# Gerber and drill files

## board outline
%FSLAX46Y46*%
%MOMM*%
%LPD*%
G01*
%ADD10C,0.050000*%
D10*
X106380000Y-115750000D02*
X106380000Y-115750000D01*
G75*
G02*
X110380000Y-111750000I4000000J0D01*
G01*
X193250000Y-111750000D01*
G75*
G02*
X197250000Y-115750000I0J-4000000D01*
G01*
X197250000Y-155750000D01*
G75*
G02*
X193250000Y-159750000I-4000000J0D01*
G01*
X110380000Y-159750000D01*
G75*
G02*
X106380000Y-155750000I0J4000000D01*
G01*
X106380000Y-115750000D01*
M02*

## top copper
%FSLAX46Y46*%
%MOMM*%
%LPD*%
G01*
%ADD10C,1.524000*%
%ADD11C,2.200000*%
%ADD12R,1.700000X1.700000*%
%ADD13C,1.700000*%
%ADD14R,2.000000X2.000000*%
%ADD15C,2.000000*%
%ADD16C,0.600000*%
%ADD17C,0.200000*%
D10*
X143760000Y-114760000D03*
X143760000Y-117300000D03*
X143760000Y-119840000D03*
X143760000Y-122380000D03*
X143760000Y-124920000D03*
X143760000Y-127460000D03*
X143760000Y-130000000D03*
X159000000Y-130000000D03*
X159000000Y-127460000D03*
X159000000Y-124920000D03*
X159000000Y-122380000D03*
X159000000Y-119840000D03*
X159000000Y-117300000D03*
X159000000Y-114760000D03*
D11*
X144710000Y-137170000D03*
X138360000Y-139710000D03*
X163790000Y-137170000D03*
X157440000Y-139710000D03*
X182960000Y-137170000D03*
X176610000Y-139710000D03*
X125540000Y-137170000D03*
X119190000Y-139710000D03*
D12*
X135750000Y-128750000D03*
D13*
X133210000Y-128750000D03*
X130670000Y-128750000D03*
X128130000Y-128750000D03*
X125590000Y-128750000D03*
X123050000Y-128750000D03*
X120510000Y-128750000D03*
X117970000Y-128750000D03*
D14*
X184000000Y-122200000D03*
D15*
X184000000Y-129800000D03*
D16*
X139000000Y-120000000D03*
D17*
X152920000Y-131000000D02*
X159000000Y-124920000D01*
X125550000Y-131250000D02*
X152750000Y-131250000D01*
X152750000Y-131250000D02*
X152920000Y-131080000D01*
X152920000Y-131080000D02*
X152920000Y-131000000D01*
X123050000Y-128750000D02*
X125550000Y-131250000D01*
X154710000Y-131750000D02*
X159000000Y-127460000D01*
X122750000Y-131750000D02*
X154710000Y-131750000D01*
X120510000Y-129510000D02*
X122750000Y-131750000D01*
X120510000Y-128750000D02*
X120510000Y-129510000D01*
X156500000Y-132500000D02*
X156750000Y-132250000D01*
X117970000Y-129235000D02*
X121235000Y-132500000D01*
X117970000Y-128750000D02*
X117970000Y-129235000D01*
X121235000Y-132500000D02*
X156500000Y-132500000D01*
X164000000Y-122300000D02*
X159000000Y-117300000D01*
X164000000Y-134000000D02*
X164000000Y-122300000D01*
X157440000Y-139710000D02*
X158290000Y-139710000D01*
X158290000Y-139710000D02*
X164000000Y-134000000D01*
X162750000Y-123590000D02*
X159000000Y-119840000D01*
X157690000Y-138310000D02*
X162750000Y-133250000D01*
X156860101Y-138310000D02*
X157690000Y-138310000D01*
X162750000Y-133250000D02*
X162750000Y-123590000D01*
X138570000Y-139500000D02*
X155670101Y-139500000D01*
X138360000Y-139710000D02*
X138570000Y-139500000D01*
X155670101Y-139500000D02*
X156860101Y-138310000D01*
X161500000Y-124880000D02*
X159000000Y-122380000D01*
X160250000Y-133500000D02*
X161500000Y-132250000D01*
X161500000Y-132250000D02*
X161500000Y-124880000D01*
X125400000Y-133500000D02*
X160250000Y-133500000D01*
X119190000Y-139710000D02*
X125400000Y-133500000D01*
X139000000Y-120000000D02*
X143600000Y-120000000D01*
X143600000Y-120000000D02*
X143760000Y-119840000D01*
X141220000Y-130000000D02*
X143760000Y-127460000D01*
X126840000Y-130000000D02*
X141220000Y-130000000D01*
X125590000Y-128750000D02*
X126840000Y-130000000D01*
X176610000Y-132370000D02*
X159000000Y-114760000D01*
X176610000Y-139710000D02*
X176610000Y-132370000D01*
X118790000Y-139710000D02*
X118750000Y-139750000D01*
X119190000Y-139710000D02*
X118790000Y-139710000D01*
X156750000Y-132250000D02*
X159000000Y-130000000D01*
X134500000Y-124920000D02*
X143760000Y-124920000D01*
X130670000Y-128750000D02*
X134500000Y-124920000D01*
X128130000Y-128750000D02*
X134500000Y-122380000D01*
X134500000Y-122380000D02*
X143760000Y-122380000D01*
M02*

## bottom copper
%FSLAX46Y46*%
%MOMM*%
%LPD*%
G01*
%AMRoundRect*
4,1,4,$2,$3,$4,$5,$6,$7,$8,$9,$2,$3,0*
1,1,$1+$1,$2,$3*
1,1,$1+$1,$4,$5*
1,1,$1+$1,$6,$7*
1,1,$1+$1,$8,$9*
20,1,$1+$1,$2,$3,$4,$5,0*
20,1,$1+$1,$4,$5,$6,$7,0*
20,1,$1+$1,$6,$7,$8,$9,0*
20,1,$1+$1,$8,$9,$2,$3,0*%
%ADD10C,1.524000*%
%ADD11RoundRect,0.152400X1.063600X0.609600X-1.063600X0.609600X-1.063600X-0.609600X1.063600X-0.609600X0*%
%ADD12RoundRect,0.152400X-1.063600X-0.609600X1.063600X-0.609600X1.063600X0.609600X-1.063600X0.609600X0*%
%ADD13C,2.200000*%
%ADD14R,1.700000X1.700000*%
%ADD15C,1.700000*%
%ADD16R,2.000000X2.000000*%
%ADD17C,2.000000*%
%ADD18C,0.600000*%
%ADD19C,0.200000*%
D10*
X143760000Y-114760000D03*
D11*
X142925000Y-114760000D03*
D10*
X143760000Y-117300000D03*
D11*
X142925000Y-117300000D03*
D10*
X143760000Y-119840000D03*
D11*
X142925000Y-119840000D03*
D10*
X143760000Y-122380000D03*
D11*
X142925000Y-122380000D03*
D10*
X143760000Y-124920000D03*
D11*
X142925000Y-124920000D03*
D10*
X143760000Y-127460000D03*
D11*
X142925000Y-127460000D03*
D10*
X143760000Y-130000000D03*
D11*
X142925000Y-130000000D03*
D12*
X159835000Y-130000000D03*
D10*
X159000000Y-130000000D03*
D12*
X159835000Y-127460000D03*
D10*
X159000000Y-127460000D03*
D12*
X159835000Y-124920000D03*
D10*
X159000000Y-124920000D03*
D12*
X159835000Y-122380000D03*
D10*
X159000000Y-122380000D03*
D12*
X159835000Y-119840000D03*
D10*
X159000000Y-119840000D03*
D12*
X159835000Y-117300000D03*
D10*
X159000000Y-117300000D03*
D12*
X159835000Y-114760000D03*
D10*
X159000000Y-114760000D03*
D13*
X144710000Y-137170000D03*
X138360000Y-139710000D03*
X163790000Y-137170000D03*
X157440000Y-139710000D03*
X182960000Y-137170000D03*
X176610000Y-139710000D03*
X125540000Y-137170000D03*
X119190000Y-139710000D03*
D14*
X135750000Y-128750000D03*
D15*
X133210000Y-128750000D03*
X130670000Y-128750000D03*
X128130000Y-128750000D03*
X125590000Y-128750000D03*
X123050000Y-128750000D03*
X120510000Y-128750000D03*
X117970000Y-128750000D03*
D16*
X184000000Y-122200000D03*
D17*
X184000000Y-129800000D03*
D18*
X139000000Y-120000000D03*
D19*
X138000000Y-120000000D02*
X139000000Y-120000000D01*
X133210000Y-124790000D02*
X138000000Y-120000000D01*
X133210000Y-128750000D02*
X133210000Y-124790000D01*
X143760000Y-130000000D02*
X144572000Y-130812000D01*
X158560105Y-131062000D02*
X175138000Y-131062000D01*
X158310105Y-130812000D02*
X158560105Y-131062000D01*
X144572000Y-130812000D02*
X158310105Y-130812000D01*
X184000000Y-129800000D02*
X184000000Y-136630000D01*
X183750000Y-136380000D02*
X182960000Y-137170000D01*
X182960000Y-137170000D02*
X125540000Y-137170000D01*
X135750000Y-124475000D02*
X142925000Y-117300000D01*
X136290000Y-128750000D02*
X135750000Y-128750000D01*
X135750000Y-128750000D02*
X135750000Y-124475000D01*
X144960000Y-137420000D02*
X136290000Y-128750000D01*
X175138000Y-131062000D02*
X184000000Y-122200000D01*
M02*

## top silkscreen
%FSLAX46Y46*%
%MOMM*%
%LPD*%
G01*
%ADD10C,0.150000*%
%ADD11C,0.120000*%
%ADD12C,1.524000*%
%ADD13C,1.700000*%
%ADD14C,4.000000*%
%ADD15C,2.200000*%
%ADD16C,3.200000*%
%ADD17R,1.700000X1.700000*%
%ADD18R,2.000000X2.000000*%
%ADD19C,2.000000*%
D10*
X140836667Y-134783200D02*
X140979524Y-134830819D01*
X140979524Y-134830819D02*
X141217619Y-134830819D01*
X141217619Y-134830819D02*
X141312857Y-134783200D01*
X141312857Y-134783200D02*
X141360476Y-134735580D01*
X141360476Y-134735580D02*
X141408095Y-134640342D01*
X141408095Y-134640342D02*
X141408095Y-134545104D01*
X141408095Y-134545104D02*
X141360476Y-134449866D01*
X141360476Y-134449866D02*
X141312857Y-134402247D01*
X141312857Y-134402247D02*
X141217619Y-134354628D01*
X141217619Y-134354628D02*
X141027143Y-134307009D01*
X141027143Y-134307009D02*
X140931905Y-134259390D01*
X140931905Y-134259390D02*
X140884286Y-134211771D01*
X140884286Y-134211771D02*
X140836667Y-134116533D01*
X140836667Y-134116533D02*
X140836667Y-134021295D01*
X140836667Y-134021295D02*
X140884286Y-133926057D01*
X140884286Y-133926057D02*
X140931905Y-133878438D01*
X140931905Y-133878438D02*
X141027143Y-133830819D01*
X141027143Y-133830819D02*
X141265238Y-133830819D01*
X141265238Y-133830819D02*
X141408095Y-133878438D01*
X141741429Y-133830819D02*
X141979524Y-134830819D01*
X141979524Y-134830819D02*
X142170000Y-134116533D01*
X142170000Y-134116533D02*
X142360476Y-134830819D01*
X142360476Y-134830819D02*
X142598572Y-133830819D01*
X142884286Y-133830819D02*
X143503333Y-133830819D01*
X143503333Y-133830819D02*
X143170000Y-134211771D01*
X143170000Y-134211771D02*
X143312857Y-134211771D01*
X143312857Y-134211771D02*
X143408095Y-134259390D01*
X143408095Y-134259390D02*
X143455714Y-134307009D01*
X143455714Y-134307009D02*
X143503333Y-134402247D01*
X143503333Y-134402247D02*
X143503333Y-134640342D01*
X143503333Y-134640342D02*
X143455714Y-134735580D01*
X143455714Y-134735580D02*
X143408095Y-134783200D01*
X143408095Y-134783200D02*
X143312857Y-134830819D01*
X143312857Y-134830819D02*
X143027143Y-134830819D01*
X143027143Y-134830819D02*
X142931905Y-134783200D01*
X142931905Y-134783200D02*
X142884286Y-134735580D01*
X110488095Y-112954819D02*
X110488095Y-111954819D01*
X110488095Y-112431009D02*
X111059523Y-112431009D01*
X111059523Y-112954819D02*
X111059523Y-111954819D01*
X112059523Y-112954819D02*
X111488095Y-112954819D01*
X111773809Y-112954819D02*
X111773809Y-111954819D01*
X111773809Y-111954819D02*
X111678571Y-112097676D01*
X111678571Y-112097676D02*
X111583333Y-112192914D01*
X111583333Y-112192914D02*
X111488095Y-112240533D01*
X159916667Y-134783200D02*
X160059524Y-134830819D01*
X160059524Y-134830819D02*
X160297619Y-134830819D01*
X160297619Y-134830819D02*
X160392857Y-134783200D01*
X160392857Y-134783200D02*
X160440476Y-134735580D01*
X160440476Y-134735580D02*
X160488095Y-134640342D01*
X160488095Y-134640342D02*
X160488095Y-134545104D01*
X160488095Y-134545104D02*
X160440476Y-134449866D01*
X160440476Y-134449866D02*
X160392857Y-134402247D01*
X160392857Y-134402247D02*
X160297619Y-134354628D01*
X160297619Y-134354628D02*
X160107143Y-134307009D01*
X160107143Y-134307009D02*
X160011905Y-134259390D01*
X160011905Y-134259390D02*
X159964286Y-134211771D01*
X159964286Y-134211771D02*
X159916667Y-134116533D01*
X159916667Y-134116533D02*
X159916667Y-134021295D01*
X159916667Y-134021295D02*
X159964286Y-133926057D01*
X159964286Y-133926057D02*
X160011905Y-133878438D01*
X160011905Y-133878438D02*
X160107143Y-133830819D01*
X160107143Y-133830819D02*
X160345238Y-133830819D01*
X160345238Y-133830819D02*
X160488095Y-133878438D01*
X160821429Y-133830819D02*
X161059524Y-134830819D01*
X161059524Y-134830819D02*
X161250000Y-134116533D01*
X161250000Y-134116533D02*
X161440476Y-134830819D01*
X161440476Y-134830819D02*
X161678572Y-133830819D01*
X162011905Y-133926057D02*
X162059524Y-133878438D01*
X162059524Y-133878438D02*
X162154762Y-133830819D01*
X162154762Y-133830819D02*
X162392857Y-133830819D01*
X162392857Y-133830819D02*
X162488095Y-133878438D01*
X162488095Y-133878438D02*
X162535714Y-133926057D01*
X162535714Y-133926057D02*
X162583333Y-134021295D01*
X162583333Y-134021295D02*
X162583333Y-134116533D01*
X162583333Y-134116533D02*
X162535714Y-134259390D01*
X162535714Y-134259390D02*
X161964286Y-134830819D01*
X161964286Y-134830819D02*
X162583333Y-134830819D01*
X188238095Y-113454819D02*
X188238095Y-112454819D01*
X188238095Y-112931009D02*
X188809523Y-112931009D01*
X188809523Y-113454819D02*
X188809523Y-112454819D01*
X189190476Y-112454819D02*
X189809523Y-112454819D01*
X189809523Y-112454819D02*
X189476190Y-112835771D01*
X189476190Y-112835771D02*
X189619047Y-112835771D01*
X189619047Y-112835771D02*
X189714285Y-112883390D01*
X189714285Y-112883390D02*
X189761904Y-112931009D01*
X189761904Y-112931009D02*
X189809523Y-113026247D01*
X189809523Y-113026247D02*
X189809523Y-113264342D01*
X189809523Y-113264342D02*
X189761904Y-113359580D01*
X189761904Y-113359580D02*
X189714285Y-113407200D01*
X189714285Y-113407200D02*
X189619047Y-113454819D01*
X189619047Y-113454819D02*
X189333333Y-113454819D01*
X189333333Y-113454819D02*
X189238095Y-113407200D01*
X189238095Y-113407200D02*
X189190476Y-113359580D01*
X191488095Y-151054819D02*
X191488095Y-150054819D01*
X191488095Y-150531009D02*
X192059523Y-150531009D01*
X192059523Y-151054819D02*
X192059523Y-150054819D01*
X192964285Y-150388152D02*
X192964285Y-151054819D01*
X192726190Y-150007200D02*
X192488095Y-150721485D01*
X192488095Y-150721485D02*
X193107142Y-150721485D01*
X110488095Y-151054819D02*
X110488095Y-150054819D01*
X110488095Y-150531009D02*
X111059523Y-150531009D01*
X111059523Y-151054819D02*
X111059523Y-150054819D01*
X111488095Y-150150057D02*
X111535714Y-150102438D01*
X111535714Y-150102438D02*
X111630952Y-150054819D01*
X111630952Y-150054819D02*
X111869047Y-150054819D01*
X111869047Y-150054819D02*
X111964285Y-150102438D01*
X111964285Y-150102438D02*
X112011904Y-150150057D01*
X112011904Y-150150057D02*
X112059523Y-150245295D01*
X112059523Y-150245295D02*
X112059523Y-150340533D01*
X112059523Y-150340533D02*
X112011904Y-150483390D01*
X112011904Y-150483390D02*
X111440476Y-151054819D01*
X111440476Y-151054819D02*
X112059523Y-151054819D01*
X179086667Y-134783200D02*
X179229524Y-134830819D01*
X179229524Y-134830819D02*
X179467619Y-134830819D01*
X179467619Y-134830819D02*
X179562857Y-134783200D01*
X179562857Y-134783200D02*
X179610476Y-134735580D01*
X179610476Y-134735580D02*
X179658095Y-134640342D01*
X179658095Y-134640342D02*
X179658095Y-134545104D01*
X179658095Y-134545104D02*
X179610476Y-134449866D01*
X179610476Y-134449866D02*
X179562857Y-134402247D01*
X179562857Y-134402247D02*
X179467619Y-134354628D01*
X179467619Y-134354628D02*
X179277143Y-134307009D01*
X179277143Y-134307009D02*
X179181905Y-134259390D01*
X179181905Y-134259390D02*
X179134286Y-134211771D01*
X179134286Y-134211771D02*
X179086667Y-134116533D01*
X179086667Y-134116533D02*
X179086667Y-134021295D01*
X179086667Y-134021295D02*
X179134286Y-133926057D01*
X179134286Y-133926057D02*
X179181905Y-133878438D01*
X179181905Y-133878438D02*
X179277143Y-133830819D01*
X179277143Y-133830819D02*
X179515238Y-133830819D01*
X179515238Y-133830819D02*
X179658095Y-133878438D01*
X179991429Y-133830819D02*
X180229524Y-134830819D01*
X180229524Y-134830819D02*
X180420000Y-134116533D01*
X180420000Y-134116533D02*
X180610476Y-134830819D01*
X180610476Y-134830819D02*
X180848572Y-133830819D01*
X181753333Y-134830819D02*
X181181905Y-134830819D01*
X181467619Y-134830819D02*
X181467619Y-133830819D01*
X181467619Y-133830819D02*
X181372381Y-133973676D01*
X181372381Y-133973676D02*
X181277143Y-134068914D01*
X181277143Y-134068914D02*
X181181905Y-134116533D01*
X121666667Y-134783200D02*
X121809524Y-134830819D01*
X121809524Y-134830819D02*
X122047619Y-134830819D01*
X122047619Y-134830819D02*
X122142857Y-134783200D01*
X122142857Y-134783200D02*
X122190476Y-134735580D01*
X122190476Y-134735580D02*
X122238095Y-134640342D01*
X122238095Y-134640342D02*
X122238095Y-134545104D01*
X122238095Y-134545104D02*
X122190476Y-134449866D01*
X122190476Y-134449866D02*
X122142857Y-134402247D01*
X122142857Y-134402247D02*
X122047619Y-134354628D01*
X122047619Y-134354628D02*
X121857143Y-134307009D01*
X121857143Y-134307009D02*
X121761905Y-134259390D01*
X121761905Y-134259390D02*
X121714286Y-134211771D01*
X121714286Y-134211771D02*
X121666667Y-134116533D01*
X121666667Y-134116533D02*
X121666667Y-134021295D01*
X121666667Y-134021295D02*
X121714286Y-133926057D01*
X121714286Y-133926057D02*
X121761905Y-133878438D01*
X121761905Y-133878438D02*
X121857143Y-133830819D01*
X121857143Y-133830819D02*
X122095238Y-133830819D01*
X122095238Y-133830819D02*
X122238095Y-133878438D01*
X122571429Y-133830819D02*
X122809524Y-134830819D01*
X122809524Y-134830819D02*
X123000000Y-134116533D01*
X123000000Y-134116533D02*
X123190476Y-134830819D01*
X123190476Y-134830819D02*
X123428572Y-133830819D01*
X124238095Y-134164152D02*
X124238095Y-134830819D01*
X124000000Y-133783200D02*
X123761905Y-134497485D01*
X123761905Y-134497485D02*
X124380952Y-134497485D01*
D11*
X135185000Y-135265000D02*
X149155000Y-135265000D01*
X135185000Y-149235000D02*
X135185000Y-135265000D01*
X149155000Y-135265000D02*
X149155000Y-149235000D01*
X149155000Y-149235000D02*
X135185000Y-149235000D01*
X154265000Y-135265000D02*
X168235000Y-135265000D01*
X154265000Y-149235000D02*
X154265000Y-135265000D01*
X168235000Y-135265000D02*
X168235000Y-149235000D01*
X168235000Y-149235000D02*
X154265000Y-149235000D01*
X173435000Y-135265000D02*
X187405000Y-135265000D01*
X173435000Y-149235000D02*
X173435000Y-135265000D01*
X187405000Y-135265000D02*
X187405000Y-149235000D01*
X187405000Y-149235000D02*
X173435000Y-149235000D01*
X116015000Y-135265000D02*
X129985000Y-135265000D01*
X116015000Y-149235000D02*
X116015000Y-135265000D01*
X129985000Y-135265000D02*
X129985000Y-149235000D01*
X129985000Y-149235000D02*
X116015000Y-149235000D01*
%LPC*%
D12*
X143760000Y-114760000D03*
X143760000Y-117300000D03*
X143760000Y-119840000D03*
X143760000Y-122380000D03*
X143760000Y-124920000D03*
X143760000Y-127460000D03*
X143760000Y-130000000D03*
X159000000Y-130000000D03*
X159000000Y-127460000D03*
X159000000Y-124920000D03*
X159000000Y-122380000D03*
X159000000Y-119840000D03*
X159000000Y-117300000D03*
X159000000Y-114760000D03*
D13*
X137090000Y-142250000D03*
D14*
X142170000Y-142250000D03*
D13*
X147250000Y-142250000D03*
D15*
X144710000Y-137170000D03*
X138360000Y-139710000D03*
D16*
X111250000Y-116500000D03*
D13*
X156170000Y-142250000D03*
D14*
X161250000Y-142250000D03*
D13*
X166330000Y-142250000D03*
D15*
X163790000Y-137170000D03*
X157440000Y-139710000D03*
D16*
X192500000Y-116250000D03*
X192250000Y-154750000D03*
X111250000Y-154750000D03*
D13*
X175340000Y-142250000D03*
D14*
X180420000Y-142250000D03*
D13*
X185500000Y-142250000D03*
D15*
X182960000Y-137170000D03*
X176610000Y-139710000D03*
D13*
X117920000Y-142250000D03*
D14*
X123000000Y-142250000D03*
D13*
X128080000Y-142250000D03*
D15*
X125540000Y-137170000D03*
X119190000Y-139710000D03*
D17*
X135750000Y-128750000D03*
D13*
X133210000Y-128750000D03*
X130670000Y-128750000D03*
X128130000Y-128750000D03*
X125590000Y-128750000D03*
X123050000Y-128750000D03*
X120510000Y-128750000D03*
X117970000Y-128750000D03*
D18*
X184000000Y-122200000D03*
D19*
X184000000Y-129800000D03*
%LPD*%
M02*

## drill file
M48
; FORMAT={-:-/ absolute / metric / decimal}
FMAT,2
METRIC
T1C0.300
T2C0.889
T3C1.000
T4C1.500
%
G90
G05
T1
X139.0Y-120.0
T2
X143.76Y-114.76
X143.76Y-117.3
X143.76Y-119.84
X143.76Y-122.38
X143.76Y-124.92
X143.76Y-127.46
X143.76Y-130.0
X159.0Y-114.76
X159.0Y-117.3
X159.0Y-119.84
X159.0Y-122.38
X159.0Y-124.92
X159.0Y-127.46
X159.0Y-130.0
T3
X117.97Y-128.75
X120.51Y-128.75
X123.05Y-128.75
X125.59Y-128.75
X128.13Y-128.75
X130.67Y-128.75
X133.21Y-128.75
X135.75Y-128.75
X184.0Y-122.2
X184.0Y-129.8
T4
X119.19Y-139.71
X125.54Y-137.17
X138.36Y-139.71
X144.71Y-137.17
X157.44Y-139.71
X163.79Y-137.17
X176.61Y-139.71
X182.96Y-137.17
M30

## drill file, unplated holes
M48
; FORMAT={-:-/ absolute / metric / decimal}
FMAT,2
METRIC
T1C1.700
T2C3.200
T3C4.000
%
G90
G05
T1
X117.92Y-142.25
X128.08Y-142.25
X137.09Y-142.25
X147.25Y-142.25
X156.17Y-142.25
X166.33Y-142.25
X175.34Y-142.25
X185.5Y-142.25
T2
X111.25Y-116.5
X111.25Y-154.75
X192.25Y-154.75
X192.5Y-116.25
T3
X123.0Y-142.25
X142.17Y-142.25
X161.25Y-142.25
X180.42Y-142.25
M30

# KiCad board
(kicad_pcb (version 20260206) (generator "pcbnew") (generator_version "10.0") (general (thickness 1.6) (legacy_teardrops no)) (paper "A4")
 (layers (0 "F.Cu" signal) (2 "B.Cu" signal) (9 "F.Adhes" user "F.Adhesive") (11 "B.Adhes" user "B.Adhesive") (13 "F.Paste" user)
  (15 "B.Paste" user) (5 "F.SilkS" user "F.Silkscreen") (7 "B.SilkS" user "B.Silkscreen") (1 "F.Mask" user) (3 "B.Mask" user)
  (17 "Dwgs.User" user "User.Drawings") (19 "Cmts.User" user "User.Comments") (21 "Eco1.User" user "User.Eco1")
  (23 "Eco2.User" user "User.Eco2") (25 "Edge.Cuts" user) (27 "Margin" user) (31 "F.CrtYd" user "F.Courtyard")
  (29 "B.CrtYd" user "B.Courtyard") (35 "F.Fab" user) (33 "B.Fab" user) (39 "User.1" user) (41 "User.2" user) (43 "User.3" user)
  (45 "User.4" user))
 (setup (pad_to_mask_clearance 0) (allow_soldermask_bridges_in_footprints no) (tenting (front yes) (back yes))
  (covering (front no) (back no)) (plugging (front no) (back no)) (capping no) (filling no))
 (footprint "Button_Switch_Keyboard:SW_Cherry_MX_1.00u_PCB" (layer "F.Cu") (at 144.71 137.17)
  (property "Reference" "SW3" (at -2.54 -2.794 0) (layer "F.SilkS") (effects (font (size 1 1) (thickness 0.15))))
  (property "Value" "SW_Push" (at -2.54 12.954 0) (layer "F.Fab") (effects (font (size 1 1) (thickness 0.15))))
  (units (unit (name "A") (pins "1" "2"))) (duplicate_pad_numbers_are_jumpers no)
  (fp_line (start -9.525 -1.905) (end 4.445 -1.905) (stroke (width 0.12) (type solid)) (layer "F.SilkS"))
  (fp_line (start -9.525 12.065) (end -9.525 -1.905) (stroke (width 0.12) (type solid)) (layer "F.SilkS"))
  (fp_line (start 4.445 -1.905) (end 4.445 12.065) (stroke (width 0.12) (type solid)) (layer "F.SilkS"))
  (fp_line (start 4.445 12.065) (end -9.525 12.065) (stroke (width 0.12) (type solid)) (layer "F.SilkS"))
  (pad "" np_thru_hole circle (at -7.62 5.08) (size 1.7 1.7) (drill 1.7) (layers "*.Cu" "*.Mask"))
  (pad "" np_thru_hole circle (at -2.54 5.08) (size 4 4) (drill 4) (layers "*.Cu" "*.Mask"))
  (pad "" np_thru_hole circle (at 2.54 5.08) (size 1.7 1.7) (drill 1.7) (layers "*.Cu" "*.Mask"))
  (pad "1" thru_hole circle (at 0 0) (size 2.2 2.2) (drill 1.5) (layers "*.Cu" "*.Mask") (remove_unused_layers no) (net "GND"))
  (pad "2" thru_hole circle (at -6.35 2.54) (size 2.2 2.2) (drill 1.5) (layers "*.Cu" "*.Mask") (remove_unused_layers no)
   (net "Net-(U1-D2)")))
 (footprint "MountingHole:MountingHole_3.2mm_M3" (layer "F.Cu") (at 111.25 116.5)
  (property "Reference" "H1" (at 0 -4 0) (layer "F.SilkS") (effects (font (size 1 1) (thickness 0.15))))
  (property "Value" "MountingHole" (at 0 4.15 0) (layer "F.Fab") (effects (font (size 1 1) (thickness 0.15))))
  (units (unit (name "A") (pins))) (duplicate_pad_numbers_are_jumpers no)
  (pad "" np_thru_hole circle (at 0 0) (size 3.2 3.2) (drill 3.2) (layers "*.Cu" "*.Mask")))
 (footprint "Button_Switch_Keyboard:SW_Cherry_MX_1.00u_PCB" (layer "F.Cu") (at 163.79 137.17)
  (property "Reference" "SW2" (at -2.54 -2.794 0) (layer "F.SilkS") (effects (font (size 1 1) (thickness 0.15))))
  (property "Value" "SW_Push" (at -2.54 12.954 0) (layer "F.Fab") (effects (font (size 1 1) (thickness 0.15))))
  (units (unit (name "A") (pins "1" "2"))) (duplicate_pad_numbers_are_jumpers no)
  (fp_line (start -9.525 -1.905) (end 4.445 -1.905) (stroke (width 0.12) (type solid)) (layer "F.SilkS"))
  (fp_line (start -9.525 12.065) (end -9.525 -1.905) (stroke (width 0.12) (type solid)) (layer "F.SilkS"))
  (fp_line (start 4.445 -1.905) (end 4.445 12.065) (stroke (width 0.12) (type solid)) (layer "F.SilkS"))
  (fp_line (start 4.445 12.065) (end -9.525 12.065) (stroke (width 0.12) (type solid)) (layer "F.SilkS"))
  (pad "" np_thru_hole circle (at -7.62 5.08) (size 1.7 1.7) (drill 1.7) (layers "*.Cu" "*.Mask"))
  (pad "" np_thru_hole circle (at -2.54 5.08) (size 4 4) (drill 4) (layers "*.Cu" "*.Mask"))
  (pad "" np_thru_hole circle (at 2.54 5.08) (size 1.7 1.7) (drill 1.7) (layers "*.Cu" "*.Mask"))
  (pad "1" thru_hole circle (at 0 0) (size 2.2 2.2) (drill 1.5) (layers "*.Cu" "*.Mask") (remove_unused_layers no) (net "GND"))
  (pad "2" thru_hole circle (at -6.35 2.54) (size 2.2 2.2) (drill 1.5) (layers "*.Cu" "*.Mask") (remove_unused_layers no)
   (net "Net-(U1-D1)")))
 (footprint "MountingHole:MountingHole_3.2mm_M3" (layer "F.Cu") (at 192.5 116.25)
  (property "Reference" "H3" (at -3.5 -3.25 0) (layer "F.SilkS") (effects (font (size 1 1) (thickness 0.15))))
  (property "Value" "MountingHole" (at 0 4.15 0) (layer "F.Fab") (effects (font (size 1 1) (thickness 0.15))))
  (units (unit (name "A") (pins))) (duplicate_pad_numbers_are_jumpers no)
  (pad "" np_thru_hole circle (at 0 0) (size 3.2 3.2) (drill 3.2) (layers "*.Cu" "*.Mask")))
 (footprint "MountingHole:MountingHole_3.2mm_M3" (layer "F.Cu") (at 192.25 154.75)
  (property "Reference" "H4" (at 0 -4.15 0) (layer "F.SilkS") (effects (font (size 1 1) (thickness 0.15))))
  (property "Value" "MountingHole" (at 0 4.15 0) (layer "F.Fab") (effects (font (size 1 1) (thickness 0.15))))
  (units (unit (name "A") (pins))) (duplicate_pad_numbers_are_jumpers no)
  (pad "" np_thru_hole circle (at 0 0) (size 3.2 3.2) (drill 3.2) (layers "*.Cu" "*.Mask")))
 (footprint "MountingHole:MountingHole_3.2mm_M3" (layer "F.Cu") (at 111.25 154.75)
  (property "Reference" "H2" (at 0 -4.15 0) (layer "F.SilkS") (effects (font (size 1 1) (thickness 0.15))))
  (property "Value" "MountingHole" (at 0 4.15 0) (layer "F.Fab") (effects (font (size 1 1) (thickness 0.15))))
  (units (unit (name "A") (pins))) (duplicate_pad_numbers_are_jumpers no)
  (pad "" np_thru_hole circle (at 0 0) (size 3.2 3.2) (drill 3.2) (layers "*.Cu" "*.Mask")))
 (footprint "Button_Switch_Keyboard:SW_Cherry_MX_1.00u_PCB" (layer "F.Cu") (at 182.96 137.17)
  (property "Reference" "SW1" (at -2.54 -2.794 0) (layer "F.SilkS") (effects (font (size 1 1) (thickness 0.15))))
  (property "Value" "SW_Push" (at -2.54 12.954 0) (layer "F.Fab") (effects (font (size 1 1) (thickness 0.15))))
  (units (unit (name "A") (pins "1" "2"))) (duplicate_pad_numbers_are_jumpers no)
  (fp_line (start -9.525 -1.905) (end 4.445 -1.905) (stroke (width 0.12) (type solid)) (layer "F.SilkS"))
  (fp_line (start -9.525 12.065) (end -9.525 -1.905) (stroke (width 0.12) (type solid)) (layer "F.SilkS"))
  (fp_line (start 4.445 -1.905) (end 4.445 12.065) (stroke (width 0.12) (type solid)) (layer "F.SilkS"))
  (fp_line (start 4.445 12.065) (end -9.525 12.065) (stroke (width 0.12) (type solid)) (layer "F.SilkS"))
  (pad "" np_thru_hole circle (at -7.62 5.08) (size 1.7 1.7) (drill 1.7) (layers "*.Cu" "*.Mask"))
  (pad "" np_thru_hole circle (at -2.54 5.08) (size 4 4) (drill 4) (layers "*.Cu" "*.Mask"))
  (pad "" np_thru_hole circle (at 2.54 5.08) (size 1.7 1.7) (drill 1.7) (layers "*.Cu" "*.Mask"))
  (pad "1" thru_hole circle (at 0 0) (size 2.2 2.2) (drill 1.5) (layers "*.Cu" "*.Mask") (remove_unused_layers no) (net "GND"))
  (pad "2" thru_hole circle (at -6.35 2.54) (size 2.2 2.2) (drill 1.5) (layers "*.Cu" "*.Mask") (remove_unused_layers no)
   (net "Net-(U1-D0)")))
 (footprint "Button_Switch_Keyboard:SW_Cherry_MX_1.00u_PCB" (layer "F.Cu") (at 125.54 137.17)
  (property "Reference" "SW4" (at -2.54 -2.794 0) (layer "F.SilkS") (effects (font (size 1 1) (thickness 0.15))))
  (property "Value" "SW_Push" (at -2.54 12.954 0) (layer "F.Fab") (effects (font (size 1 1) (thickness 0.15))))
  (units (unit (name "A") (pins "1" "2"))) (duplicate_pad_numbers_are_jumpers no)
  (fp_line (start -9.525 -1.905) (end 4.445 -1.905) (stroke (width 0.12) (type solid)) (layer "F.SilkS"))
  (fp_line (start -9.525 12.065) (end -9.525 -1.905) (stroke (width 0.12) (type solid)) (layer "F.SilkS"))
  (fp_line (start 4.445 -1.905) (end 4.445 12.065) (stroke (width 0.12) (type solid)) (layer "F.SilkS"))
  (fp_line (start 4.445 12.065) (end -9.525 12.065) (stroke (width 0.12) (type solid)) (layer "F.SilkS"))
  (pad "" np_thru_hole circle (at -7.62 5.08) (size 1.7 1.7) (drill 1.7) (layers "*.Cu" "*.Mask"))
  (pad "" np_thru_hole circle (at -2.54 5.08) (size 4 4) (drill 4) (layers "*.Cu" "*.Mask"))
  (pad "" np_thru_hole circle (at 2.54 5.08) (size 1.7 1.7) (drill 1.7) (layers "*.Cu" "*.Mask"))
  (pad "1" thru_hole circle (at 0 0) (size 2.2 2.2) (drill 1.5) (layers "*.Cu" "*.Mask") (remove_unused_layers no) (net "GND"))
  (pad "2" thru_hole circle (at -6.35 2.54) (size 2.2 2.2) (drill 1.5) (layers "*.Cu" "*.Mask") (remove_unused_layers no)
   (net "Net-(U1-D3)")))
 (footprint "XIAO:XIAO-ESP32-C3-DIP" (layer "B.Cu") (at 151.38 122.38 90)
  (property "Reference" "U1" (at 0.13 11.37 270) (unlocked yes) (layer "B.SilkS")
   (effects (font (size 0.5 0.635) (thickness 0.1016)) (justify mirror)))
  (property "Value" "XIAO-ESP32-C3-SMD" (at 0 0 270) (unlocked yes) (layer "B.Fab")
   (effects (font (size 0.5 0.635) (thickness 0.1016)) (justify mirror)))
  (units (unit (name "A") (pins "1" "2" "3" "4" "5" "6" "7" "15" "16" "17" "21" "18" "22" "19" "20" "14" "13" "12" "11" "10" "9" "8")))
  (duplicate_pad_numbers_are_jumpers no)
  (pad "1" thru_hole circle (at 7.62 7.62) (size 1.524 1.524) (drill 0.889) (layers "*.Cu" "*.Mask") (remove_unused_layers no)
   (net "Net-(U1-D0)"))
  (pad "1" smd roundrect (at 7.62 8.455) (size 2.432 1.524) (layers "B.Cu" "B.Mask") (roundrect_rratio 0.1) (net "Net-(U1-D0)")
   (thermal_bridge_angle 45))
  (pad "2" thru_hole circle (at 5.08 7.62) (size 1.524 1.524) (drill 0.889) (layers "*.Cu" "*.Mask") (remove_unused_layers no)
   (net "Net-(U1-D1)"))
  (pad "2" smd roundrect (at 5.08 8.455) (size 2.432 1.524) (layers "B.Cu" "B.Mask") (roundrect_rratio 0.1) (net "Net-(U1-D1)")
   (thermal_bridge_angle 45))
  (pad "3" thru_hole circle (at 2.54 7.62) (size 1.524 1.524) (drill 0.889) (layers "*.Cu" "*.Mask") (remove_unused_layers no)
   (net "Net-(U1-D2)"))
  (pad "3" smd roundrect (at 2.54 8.455) (size 2.432 1.524) (layers "B.Cu" "B.Mask") (roundrect_rratio 0.1) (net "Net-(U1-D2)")
   (thermal_bridge_angle 45))
  (pad "4" thru_hole circle (at 0 7.62) (size 1.524 1.524) (drill 0.889) (layers "*.Cu" "*.Mask") (remove_unused_layers no)
   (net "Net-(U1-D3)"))
  (pad "4" smd roundrect (at 0 8.455) (size 2.432 1.524) (layers "B.Cu" "B.Mask") (roundrect_rratio 0.1) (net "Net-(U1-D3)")
   (thermal_bridge_angle 45))
  (pad "5" thru_hole circle (at -2.54 7.62) (size 1.524 1.524) (drill 0.889) (layers "*.Cu" "*.Mask") (remove_unused_layers no) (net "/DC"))
  (pad "5" smd roundrect (at -2.54 8.455) (size 2.432 1.524) (layers "B.Cu" "B.Mask") (roundrect_rratio 0.1) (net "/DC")
   (thermal_bridge_angle 45))
  (pad "6" thru_hole circle (at -5.08 7.62) (size 1.524 1.524) (drill 0.889) (layers "*.Cu" "*.Mask") (remove_unused_layers no) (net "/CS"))
  (pad "6" smd roundrect (at -5.08 8.455) (size 2.432 1.524) (layers "B.Cu" "B.Mask") (roundrect_rratio 0.1) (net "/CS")
   (thermal_bridge_angle 45))
  (pad "7" thru_hole circle (at -7.62 7.62) (size 1.524 1.524) (drill 0.889) (layers "*.Cu" "*.Mask") (remove_unused_layers no) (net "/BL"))
  (pad "7" smd roundrect (at -7.62 8.455) (size 2.432 1.524) (layers "B.Cu" "B.Mask") (roundrect_rratio 0.1) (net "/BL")
   (thermal_bridge_angle 45))
  (pad "8" smd roundrect (at -7.62 -8.455 180) (size 2.432 1.524) (layers "B.Cu" "B.Mask") (roundrect_rratio 0.1) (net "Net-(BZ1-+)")
   (thermal_bridge_angle 45))
  (pad "8" thru_hole circle (at -7.62 -7.62 180) (size 1.524 1.524) (drill 0.889) (layers "*.Cu" "*.Mask") (remove_unused_layers no)
   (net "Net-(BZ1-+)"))
  (pad "9" smd roundrect (at -5.08 -8.455 180) (size 2.432 1.524) (layers "B.Cu" "B.Mask") (roundrect_rratio 0.1) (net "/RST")
   (thermal_bridge_angle 45))
  (pad "9" thru_hole circle (at -5.08 -7.62 180) (size 1.524 1.524) (drill 0.889) (layers "*.Cu" "*.Mask") (remove_unused_layers no)
   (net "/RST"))
  (pad "10" smd roundrect (at -2.54 -8.455 180) (size 2.432 1.524) (layers "B.Cu" "B.Mask") (roundrect_rratio 0.1) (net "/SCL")
   (thermal_bridge_angle 45))
  (pad "10" thru_hole circle (at -2.54 -7.62 180) (size 1.524 1.524) (drill 0.889) (layers "*.Cu" "*.Mask") (remove_unused_layers no)
   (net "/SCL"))
  (pad "11" smd roundrect (at 0 -8.455 180) (size 2.432 1.524) (layers "B.Cu" "B.Mask") (roundrect_rratio 0.1) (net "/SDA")
   (thermal_bridge_angle 45))
  (pad "11" thru_hole circle (at 0 -7.62 180) (size 1.524 1.524) (drill 0.889) (layers "*.Cu" "*.Mask") (remove_unused_layers no)
   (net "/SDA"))
  (pad "12" smd roundrect (at 2.54 -8.455 180) (size 2.432 1.524) (layers "B.Cu" "B.Mask") (roundrect_rratio 0.1) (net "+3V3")
   (thermal_bridge_angle 45))
  (pad "12" thru_hole circle (at 2.54 -7.62 180) (size 1.524 1.524) (drill 0.889) (layers "*.Cu" "*.Mask") (remove_unused_layers no)
   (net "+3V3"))
  (pad "13" smd roundrect (at 5.08 -8.455 180) (size 2.432 1.524) (layers "B.Cu" "B.Mask") (roundrect_rratio 0.1) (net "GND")
   (thermal_bridge_angle 45))
  (pad "13" thru_hole circle (at 5.08 -7.62 180) (size 1.524 1.524) (drill 0.889) (layers "*.Cu" "*.Mask") (remove_unused_layers no)
   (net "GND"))
  (pad "14" smd roundrect (at 7.62 -8.455 180) (size 2.432 1.524) (layers "B.Cu" "B.Mask") (roundrect_rratio 0.1)
   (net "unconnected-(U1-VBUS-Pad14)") (thermal_bridge_angle 45))
  (pad "14" thru_hole circle (at 7.62 -7.62 180) (size 1.524 1.524) (drill 0.889) (layers "*.Cu" "*.Mask") (remove_unused_layers no)
   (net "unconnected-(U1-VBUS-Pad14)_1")))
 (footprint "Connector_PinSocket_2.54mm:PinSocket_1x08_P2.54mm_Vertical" (layer "B.Cu") (at 135.75 128.75 90)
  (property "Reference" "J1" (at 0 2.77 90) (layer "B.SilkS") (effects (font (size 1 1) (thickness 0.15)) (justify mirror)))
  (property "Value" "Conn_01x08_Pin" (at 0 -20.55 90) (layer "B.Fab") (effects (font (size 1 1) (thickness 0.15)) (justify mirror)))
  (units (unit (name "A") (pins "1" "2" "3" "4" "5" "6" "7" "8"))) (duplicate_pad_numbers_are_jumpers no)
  (pad "1" thru_hole rect (at 0 0 90) (size 1.7 1.7) (drill 1) (layers "*.Cu" "*.Mask") (remove_unused_layers no) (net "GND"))
  (pad "2" thru_hole circle (at 0 -2.54 90) (size 1.7 1.7) (drill 1) (layers "*.Cu" "*.Mask") (remove_unused_layers no) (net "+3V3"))
  (pad "3" thru_hole circle (at 0 -5.08 90) (size 1.7 1.7) (drill 1) (layers "*.Cu" "*.Mask") (remove_unused_layers no) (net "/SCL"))
  (pad "4" thru_hole circle (at 0 -7.62 90) (size 1.7 1.7) (drill 1) (layers "*.Cu" "*.Mask") (remove_unused_layers no) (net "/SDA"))
  (pad "5" thru_hole circle (at 0 -10.16 90) (size 1.7 1.7) (drill 1) (layers "*.Cu" "*.Mask") (remove_unused_layers no) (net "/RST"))
  (pad "6" thru_hole circle (at 0 -12.7 90) (size 1.7 1.7) (drill 1) (layers "*.Cu" "*.Mask") (remove_unused_layers no) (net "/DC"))
  (pad "7" thru_hole circle (at 0 -15.24 90) (size 1.7 1.7) (drill 1) (layers "*.Cu" "*.Mask") (remove_unused_layers no) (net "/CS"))
  (pad "8" thru_hole circle (at 0 -17.78 90) (size 1.7 1.7) (drill 1) (layers "*.Cu" "*.Mask") (remove_unused_layers no) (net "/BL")))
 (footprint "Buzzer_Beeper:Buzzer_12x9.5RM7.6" (layer "B.Cu") (at 184 122.2 -90)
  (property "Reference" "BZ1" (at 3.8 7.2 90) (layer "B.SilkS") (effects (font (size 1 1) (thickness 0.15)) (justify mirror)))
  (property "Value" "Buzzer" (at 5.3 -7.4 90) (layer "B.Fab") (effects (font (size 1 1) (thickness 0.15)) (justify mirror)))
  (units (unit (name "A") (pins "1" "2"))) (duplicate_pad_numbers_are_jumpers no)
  (pad "1" thru_hole rect (at 0 0 270) (size 2 2) (drill 1) (layers "*.Cu" "*.Mask") (remove_unused_layers no) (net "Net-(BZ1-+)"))
  (pad "2" thru_hole circle (at 7.6 0 270) (size 2 2) (drill 1) (layers "*.Cu" "*.Mask") (remove_unused_layers no) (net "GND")))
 (gr_rect (start 106.38 111.75) (end 197.25 159.75) (radius 4) (stroke (width 0.05) (type default)) (fill no) (layer "Edge.Cuts"))
 (segment (start 184 129.8) (end 184 136.63) (width 0.2) (layer "B.Cu") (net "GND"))
 (segment (start 183.75 136.38) (end 182.96 137.17) (width 0.2) (layer "B.Cu") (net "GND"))
 (segment (start 182.96 137.17) (end 125.54 137.17) (width 0.2) (layer "B.Cu") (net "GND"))
 (segment (start 135.75 124.475) (end 142.925 117.3) (width 0.2) (layer "B.Cu") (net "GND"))
 (segment (start 136.29 128.75) (end 135.75 128.75) (width 0.2) (layer "B.Cu") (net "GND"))
 (segment (start 135.75 128.75) (end 135.75 124.475) (width 0.2) (layer "B.Cu") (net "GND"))
 (segment (start 144.96 137.42) (end 136.29 128.75) (width 0.2) (layer "B.Cu") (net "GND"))
 (segment (start 156.860101 138.31) (end 157.69 138.31) (width 0.2) (layer "F.Cu") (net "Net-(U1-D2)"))
 (segment (start 138.36 139.71) (end 138.57 139.5) (width 0.2) (layer "F.Cu") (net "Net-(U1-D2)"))
 (segment (start 155.670101 139.5) (end 156.860101 138.31) (width 0.2) (layer "F.Cu") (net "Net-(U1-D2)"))
 (segment (start 162.75 133.25) (end 162.75 123.59) (width 0.2) (layer "F.Cu") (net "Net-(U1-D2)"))
 (segment (start 138.57 139.5) (end 155.670101 139.5) (width 0.2) (layer "F.Cu") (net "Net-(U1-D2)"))
 (segment (start 157.69 138.31) (end 162.75 133.25) (width 0.2) (layer "F.Cu") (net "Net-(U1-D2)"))
 (segment (start 162.75 123.59) (end 159 119.84) (width 0.2) (layer "F.Cu") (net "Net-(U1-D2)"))
 (segment (start 164 122.3) (end 159 117.3) (width 0.2) (layer "F.Cu") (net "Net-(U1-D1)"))
 (segment (start 158.29 139.71) (end 164 134) (width 0.2) (layer "F.Cu") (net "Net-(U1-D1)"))
 (segment (start 164 134) (end 164 122.3) (width 0.2) (layer "F.Cu") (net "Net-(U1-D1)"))
 (segment (start 157.44 139.71) (end 158.29 139.71) (width 0.2) (layer "F.Cu") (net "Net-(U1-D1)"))
 (segment (start 176.61 139.71) (end 176.61 132.37) (width 0.2) (layer "F.Cu") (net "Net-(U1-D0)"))
 (segment (start 176.61 132.37) (end 159 114.76) (width 0.2) (layer "F.Cu") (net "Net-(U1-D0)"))
 (segment (start 161.5 124.88) (end 159 122.38) (width 0.2) (layer "F.Cu") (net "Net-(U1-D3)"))
 (segment (start 160.25 133.5) (end 161.5 132.25) (width 0.2) (layer "F.Cu") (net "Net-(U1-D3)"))
 (segment (start 119.19 139.71) (end 125.4 133.5) (width 0.2) (layer "F.Cu") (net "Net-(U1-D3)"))
 (segment (start 161.5 132.25) (end 161.5 124.88) (width 0.2) (layer "F.Cu") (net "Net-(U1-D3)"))
 (segment (start 125.4 133.5) (end 160.25 133.5) (width 0.2) (layer "F.Cu") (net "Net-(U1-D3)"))
 (segment (start 118.79 139.71) (end 118.75 139.75) (width 0.2) (layer "F.Cu") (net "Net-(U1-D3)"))
 (segment (start 119.19 139.71) (end 118.79 139.71) (width 0.2) (layer "F.Cu") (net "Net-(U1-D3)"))
 (segment (start 152.92 131.08) (end 152.92 131) (width 0.2) (layer "F.Cu") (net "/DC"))
 (segment (start 125.55 131.25) (end 152.75 131.25) (width 0.2) (layer "F.Cu") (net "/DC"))
 (segment (start 152.75 131.25) (end 152.92 131.08) (width 0.2) (layer "F.Cu") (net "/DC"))
 (segment (start 123.05 128.75) (end 125.55 131.25) (width 0.2) (layer "F.Cu") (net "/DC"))
 (segment (start 152.92 131) (end 159 124.92) (width 0.2) (layer "F.Cu") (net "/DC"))
 (segment (start 120.51 129.51) (end 122.75 131.75) (width 0.2) (layer "F.Cu") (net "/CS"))
 (segment (start 120.51 128.75) (end 120.51 129.51) (width 0.2) (layer "F.Cu") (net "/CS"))
 (segment (start 154.71 131.75) (end 159 127.46) (width 0.2) (layer "F.Cu") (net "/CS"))
 (segment (start 122.75 131.75) (end 154.71 131.75) (width 0.2) (layer "F.Cu") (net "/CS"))
 (segment (start 156.5 132.5) (end 156.75 132.25) (width 0.2) (layer "F.Cu") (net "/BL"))
 (segment (start 121.235 132.5) (end 156.5 132.5) (width 0.2) (layer "F.Cu") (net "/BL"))
 (segment (start 156.75 132.25) (end 159 130) (width 0.2) (layer "F.Cu") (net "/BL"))
 (segment (start 117.97 129.235) (end 121.235 132.5) (width 0.2) (layer "F.Cu") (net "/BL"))
 (segment (start 117.97 128.75) (end 117.97 129.235) (width 0.2) (layer "F.Cu") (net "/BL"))
 (segment (start 158.310105 130.812) (end 158.560105 131.062) (width 0.2) (layer "B.Cu") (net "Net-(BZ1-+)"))
 (segment (start 143.76 130) (end 144.572 130.812) (width 0.2) (layer "B.Cu") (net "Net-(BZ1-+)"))
 (segment (start 175.138 131.062) (end 184 122.2) (width 0.2) (layer "B.Cu") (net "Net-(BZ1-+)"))
 (segment (start 158.560105 131.062) (end 175.138 131.062) (width 0.2) (layer "B.Cu") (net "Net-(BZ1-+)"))
 (segment (start 144.572 130.812) (end 158.310105 130.812) (width 0.2) (layer "B.Cu") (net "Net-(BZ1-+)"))
 (segment (start 125.59 128.75) (end 126.84 130) (width 0.2) (layer "F.Cu") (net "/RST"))
 (segment (start 126.84 130) (end 141.22 130) (width 0.2) (layer "F.Cu") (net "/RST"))
 (segment (start 141.22 130) (end 143.76 127.46) (width 0.2) (layer "F.Cu") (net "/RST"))
 (segment (start 134.5 124.92) (end 143.76 124.92) (width 0.2) (layer "F.Cu") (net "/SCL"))
 (segment (start 130.67 128.75) (end 134.5 124.92) (width 0.2) (layer "F.Cu") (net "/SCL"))
 (segment (start 128.13 128.75) (end 134.5 122.38) (width 0.2) (layer "F.Cu") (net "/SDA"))
 (segment (start 134.5 122.38) (end 143.76 122.38) (width 0.2) (layer "F.Cu") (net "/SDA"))
 (segment (start 143.6 120) (end 143.76 119.84) (width 0.2) (layer "F.Cu") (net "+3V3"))
 (segment (start 139 120) (end 143.6 120) (width 0.2) (layer "F.Cu") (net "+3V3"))
 (via (at 139 120) (size 0.6) (drill 0.3) (layers "F.Cu" "B.Cu") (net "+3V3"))
 (segment (start 133.21 128.75) (end 133.21 124.79) (width 0.2) (layer "B.Cu") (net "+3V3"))
 (segment (start 138 120) (end 139 120) (width 0.2) (layer "B.Cu") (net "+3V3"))
 (segment (start 133.21 124.79) (end 138 120) (width 0.2) (layer "B.Cu") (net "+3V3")))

